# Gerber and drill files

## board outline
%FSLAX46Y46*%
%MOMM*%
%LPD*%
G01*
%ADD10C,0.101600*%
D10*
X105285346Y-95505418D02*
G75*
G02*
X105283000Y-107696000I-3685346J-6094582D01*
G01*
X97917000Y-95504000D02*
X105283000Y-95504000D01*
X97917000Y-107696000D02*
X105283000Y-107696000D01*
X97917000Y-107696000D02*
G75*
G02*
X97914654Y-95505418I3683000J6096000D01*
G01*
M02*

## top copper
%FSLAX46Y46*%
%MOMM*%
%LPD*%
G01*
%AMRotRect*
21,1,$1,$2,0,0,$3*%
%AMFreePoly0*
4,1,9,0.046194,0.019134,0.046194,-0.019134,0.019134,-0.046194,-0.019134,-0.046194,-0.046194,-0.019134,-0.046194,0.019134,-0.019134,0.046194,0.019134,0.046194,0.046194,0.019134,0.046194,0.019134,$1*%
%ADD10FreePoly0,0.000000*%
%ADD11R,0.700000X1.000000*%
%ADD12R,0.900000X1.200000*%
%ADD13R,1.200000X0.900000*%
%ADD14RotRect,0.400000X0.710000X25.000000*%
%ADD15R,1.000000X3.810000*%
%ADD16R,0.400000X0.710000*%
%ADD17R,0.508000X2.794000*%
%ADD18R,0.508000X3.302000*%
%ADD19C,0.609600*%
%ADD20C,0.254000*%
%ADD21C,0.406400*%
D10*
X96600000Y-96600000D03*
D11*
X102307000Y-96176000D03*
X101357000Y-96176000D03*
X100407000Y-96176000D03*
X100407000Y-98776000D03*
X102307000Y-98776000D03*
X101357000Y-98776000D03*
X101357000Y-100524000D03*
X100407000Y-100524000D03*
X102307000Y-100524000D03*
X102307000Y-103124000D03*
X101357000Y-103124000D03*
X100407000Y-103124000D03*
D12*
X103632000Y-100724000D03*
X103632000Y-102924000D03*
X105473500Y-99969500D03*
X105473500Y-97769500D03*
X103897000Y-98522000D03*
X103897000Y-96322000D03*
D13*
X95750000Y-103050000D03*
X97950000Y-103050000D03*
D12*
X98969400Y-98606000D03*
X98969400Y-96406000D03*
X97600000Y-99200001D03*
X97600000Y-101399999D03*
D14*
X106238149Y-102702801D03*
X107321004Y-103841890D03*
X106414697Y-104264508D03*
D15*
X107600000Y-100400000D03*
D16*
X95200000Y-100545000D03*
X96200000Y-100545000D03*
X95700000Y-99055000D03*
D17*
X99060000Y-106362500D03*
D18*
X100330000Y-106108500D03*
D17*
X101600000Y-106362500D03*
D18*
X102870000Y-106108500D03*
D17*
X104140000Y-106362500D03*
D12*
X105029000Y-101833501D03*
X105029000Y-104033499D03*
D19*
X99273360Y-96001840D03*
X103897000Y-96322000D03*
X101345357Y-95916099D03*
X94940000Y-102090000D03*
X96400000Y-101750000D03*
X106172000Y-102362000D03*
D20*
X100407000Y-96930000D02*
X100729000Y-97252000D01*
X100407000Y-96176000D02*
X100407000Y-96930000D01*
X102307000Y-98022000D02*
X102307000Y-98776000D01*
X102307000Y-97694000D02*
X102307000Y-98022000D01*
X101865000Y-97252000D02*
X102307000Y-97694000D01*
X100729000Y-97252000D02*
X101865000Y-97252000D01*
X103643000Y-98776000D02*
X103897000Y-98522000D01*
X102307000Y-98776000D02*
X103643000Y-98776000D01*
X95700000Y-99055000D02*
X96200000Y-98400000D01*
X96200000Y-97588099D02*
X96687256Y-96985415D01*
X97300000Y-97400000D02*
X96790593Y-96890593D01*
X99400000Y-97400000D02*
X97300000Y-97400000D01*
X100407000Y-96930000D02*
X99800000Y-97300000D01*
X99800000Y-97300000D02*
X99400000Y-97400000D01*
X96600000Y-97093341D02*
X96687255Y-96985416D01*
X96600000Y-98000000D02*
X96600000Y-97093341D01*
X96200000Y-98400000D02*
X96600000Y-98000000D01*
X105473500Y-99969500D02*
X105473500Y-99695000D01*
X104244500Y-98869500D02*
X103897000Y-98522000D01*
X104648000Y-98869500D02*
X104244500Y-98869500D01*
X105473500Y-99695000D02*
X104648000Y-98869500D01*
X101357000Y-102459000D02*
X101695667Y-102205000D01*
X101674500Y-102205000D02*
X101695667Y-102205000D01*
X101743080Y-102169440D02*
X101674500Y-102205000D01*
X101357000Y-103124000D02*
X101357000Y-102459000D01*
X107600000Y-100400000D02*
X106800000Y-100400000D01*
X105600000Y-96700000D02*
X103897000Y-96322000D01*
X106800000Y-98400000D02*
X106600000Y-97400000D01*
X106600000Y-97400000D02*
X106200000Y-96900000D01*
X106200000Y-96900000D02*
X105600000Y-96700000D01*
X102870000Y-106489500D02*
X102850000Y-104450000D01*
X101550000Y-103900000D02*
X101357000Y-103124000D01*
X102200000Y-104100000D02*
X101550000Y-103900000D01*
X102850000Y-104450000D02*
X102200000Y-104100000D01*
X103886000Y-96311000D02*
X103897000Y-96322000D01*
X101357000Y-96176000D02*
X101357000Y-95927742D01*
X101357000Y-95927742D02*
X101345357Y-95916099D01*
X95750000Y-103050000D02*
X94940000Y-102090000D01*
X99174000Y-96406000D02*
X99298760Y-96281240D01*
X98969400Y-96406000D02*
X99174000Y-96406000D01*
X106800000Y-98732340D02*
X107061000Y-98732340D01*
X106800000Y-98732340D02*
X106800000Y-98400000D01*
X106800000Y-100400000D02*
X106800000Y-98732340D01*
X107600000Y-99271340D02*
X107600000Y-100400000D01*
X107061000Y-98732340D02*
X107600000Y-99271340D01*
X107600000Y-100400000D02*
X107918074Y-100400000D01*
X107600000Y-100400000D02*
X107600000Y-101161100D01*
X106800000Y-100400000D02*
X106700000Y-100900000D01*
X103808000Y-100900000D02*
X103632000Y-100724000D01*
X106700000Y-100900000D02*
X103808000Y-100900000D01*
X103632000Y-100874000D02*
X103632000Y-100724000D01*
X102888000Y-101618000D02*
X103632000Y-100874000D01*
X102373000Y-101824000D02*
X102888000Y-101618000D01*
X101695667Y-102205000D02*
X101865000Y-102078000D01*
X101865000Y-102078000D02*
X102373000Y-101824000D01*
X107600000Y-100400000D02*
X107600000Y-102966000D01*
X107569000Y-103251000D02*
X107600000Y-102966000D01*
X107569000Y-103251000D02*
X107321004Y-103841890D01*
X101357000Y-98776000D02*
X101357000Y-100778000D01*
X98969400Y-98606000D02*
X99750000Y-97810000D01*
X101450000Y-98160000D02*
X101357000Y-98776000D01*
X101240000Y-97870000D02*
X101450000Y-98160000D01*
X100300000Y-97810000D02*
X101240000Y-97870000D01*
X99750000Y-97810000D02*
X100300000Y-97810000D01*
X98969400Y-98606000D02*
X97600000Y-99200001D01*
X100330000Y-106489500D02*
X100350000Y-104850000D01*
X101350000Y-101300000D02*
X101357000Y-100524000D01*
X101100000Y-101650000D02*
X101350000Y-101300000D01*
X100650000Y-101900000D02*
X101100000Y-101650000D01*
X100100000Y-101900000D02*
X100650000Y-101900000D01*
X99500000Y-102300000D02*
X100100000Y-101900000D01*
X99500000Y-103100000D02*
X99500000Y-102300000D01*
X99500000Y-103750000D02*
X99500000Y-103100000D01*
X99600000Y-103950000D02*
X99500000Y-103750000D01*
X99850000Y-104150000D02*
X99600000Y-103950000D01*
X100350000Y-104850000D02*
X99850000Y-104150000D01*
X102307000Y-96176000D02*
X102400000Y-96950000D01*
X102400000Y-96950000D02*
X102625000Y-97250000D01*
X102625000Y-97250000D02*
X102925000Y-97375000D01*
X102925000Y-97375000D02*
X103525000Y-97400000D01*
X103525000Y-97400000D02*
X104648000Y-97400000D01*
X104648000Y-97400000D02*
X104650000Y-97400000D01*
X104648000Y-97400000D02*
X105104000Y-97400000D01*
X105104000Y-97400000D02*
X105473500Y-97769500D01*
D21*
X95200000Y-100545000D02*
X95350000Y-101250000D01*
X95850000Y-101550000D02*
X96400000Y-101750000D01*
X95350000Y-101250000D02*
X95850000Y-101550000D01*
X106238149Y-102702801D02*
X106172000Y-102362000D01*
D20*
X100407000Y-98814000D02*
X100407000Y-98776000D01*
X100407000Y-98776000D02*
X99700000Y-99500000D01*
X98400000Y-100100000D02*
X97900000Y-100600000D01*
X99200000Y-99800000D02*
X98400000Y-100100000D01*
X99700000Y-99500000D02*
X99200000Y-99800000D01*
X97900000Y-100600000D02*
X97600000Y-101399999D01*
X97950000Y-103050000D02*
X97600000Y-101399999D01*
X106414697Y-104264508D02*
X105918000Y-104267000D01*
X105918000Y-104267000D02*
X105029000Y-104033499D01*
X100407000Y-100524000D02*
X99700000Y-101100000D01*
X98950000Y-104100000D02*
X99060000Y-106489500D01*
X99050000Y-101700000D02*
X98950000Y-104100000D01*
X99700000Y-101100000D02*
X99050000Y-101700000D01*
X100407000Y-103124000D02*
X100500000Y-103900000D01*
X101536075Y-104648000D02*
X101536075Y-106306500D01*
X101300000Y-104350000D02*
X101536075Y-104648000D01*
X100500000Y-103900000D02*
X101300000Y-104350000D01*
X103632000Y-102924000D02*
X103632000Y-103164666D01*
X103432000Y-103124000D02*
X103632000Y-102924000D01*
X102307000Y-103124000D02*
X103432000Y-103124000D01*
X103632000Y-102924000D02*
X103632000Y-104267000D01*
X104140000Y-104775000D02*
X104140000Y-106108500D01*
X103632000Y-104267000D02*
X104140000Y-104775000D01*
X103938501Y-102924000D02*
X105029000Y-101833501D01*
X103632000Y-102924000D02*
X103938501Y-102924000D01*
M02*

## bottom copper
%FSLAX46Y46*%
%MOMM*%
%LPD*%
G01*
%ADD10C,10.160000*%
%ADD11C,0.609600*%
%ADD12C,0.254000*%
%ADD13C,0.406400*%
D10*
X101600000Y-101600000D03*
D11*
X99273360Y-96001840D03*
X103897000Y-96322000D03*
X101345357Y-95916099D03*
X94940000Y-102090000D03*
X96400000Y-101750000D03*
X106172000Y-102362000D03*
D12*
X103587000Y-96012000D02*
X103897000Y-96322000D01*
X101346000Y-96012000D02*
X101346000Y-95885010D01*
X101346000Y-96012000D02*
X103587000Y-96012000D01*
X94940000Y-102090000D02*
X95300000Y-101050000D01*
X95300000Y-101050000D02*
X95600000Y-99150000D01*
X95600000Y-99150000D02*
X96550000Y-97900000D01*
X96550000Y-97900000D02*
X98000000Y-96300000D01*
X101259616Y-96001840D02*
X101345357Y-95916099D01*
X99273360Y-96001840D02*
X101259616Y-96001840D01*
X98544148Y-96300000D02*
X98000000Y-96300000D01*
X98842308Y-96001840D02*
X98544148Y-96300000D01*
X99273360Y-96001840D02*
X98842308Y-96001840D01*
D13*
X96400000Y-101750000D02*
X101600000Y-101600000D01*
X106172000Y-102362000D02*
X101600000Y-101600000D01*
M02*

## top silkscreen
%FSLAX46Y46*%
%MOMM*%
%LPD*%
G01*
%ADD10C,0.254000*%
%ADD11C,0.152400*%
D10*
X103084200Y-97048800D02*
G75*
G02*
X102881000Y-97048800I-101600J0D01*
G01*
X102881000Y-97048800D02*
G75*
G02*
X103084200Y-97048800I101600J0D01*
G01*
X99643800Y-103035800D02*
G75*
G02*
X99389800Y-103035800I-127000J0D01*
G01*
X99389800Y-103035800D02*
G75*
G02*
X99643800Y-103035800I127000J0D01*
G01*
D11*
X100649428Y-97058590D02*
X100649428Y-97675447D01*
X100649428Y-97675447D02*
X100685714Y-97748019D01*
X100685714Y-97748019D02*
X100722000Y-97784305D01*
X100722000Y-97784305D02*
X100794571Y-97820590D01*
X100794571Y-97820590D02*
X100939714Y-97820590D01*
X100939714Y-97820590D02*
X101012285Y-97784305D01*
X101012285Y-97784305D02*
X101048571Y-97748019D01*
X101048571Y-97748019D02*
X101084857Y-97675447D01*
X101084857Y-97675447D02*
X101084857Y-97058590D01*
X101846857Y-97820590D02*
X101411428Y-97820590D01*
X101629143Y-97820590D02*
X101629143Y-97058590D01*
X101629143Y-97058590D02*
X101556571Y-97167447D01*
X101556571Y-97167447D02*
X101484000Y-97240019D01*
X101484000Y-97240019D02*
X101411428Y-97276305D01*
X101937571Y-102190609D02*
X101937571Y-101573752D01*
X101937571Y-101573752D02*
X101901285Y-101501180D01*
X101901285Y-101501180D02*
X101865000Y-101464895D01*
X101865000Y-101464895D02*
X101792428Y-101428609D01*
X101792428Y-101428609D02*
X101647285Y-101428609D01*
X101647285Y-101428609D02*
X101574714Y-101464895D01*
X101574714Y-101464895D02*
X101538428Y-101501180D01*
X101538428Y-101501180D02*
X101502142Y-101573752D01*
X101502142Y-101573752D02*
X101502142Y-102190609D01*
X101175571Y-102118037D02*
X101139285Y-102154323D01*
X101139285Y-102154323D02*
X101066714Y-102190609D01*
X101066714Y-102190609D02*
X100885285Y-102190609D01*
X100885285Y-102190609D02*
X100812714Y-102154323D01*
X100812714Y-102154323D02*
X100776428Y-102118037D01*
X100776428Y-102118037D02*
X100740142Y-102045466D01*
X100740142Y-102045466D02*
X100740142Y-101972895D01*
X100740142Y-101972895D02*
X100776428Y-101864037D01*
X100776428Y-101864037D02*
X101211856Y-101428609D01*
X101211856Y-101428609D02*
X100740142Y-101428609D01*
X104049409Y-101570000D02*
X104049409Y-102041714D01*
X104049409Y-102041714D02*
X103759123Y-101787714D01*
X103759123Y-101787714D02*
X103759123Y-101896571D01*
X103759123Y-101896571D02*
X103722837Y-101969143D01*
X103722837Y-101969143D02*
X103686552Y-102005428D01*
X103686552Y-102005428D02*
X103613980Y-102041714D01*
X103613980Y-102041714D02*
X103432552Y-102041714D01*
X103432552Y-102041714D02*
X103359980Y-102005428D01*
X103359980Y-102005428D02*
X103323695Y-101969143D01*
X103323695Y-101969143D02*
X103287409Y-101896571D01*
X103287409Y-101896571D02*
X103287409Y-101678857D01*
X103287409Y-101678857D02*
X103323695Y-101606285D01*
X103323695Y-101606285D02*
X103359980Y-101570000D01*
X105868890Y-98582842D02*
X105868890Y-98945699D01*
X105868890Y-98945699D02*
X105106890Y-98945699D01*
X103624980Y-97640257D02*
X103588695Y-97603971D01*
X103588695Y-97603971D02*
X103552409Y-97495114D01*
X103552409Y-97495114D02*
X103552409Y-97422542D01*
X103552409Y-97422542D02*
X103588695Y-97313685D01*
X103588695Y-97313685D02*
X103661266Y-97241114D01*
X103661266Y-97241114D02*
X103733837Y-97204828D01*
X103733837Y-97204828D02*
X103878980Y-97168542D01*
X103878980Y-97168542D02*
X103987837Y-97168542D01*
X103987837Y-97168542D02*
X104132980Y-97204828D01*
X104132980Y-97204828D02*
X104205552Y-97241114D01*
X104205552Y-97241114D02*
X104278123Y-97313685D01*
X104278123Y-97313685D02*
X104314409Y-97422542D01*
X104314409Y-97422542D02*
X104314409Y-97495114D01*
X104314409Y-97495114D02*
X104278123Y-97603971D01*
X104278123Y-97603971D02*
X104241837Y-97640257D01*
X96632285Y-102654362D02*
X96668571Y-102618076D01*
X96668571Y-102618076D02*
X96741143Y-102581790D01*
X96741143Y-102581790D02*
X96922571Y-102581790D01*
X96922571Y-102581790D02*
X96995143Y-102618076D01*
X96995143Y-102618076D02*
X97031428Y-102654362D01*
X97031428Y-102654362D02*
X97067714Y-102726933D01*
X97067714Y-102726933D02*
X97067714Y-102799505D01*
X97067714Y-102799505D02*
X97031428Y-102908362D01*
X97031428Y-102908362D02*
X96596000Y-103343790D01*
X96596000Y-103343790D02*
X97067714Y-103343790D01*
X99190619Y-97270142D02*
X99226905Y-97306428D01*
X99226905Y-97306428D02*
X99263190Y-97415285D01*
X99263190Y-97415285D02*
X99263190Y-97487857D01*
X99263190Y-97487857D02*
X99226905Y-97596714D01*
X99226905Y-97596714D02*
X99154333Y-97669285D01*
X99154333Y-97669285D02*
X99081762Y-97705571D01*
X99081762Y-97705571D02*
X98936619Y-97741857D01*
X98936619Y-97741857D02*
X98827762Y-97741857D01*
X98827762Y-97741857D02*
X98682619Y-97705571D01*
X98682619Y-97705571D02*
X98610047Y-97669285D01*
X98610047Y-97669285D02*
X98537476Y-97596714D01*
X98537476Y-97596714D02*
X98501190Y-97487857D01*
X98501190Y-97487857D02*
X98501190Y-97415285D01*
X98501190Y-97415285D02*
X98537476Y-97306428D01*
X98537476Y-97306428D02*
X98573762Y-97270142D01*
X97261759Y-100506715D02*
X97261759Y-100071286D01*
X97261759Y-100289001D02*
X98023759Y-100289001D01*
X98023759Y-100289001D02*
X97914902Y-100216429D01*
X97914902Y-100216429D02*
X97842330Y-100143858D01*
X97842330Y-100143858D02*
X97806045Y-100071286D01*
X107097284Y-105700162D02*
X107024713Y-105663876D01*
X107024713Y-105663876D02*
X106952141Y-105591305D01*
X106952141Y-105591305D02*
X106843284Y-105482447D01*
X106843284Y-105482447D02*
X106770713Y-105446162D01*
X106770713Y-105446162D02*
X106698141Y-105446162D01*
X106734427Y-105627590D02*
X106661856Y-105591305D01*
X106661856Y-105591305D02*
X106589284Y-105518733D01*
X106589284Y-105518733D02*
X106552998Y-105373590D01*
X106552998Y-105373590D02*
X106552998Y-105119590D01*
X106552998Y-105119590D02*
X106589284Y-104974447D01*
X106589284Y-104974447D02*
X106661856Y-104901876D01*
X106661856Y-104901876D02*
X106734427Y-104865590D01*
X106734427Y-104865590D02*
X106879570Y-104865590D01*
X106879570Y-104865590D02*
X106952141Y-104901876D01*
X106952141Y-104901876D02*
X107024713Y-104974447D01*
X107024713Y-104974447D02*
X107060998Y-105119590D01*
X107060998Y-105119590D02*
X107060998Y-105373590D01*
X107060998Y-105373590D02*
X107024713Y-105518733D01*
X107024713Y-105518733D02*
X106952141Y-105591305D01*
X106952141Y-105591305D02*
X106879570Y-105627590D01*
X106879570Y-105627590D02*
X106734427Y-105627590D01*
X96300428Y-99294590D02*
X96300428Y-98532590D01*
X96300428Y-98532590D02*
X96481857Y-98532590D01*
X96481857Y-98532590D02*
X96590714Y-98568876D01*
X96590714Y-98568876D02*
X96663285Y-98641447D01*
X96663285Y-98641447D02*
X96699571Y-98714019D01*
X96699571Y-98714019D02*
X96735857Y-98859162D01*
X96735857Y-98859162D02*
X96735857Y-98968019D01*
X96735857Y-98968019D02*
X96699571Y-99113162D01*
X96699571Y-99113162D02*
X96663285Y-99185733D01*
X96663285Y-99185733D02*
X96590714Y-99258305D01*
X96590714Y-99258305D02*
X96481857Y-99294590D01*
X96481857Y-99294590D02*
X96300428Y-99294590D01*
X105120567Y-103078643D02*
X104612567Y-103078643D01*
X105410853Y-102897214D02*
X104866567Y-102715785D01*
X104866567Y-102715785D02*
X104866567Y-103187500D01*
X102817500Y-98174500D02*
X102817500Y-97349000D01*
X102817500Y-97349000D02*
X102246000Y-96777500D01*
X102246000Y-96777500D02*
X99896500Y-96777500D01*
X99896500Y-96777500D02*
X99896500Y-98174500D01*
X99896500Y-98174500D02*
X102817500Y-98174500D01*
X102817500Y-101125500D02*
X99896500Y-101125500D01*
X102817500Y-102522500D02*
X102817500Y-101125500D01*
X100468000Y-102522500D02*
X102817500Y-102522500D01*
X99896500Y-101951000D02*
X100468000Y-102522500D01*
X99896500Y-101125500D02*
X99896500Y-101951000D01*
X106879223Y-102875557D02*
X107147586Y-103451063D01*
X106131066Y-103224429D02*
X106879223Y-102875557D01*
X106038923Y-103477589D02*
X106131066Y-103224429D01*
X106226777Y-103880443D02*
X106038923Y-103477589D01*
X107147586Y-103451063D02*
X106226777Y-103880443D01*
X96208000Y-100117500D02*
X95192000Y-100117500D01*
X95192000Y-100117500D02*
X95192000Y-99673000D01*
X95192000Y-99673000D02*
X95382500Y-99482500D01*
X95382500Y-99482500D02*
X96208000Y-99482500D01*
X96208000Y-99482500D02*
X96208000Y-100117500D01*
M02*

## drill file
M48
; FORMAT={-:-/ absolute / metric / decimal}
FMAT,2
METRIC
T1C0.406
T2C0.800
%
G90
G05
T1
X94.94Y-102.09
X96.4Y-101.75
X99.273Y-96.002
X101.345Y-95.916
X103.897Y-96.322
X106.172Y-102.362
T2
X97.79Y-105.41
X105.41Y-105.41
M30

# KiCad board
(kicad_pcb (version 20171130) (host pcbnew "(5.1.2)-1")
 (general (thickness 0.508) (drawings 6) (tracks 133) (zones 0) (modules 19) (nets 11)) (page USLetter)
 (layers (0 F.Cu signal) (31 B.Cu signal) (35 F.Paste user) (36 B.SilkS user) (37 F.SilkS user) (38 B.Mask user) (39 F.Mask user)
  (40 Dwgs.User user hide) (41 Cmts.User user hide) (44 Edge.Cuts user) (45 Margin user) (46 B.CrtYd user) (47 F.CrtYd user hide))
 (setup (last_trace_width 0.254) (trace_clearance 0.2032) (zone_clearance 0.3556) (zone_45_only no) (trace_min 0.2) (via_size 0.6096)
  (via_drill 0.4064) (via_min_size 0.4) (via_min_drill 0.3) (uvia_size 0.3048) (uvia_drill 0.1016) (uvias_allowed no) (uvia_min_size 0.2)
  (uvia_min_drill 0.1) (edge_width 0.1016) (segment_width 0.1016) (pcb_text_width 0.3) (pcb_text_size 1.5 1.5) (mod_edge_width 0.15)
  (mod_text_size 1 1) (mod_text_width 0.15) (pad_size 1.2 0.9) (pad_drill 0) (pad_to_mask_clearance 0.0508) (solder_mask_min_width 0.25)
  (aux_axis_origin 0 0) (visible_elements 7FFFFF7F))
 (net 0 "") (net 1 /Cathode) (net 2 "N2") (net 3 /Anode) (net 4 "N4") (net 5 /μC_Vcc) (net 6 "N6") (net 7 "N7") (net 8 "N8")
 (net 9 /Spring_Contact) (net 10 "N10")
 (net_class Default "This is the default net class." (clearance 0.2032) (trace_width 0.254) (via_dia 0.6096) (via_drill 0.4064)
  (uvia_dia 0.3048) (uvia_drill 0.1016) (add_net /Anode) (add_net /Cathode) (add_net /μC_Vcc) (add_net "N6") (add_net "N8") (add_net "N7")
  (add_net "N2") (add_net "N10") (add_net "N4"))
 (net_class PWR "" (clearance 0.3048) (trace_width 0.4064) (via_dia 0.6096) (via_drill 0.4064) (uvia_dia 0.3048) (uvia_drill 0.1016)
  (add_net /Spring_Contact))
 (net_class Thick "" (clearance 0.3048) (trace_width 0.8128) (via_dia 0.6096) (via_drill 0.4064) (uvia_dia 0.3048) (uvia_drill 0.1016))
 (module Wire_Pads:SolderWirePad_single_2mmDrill (layer F.Cu) (at 105.41 105.41)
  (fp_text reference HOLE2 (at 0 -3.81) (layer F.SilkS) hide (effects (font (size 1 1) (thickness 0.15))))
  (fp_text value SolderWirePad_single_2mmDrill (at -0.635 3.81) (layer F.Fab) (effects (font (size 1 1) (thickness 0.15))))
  (pad "" np_thru_hole circle (at 0 0) (size 0.8 0.8) (drill 0.8) (layers *.Cu *.Mask)))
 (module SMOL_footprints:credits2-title (layer B.Cu) (at 101.6 101.727 100)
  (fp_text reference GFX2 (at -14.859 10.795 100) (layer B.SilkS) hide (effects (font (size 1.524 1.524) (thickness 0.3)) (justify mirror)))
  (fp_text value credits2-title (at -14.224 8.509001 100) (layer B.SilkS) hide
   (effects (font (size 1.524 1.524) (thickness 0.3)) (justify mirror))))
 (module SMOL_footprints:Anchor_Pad (layer F.Cu) (at 96.5 96.6)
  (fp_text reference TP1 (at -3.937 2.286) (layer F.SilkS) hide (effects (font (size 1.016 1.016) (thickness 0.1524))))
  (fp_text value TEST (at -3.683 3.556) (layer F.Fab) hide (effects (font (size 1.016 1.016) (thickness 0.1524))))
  (pad 1 smd custom (at 0.1 0) (size 0.1 0.1) (layers F.Cu F.Mask) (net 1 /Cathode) (zone_connect 0)
   (options (clearance outline) (anchor circle)) (primitives)))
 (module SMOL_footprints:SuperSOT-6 (layer F.Cu) (at 101.357 97.476 270)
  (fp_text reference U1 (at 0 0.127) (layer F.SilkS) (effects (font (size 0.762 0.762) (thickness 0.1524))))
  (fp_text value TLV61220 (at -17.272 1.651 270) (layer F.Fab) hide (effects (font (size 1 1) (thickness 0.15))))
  (fp_line (start 0.6985 -1.4605) (end -0.127 -1.4605) (layer F.SilkS) (width 0.1524))
  (fp_line (start -0.127 -1.4605) (end -0.6985 -0.889) (layer F.SilkS) (width 0.1524))
  (fp_line (start -0.6985 -0.889) (end -0.6985 1.4605) (layer F.SilkS) (width 0.1524))
  (fp_line (start -0.6985 1.4605) (end 0.6985 1.4605) (layer F.SilkS) (width 0.1524))
  (fp_line (start 0.6985 1.4605) (end 0.6985 -1.4605) (layer F.SilkS) (width 0.1524))
  (pad 1 smd rect (at -1.3 -0.95 270) (size 1 0.7) (layers F.Cu F.Paste F.Mask) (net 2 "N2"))
  (pad 2 smd rect (at -1.3 0 270) (size 1 0.7) (layers F.Cu F.Paste F.Mask) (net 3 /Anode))
  (pad 3 smd rect (at -1.3 0.95 270) (size 1 0.7) (layers F.Cu F.Paste F.Mask) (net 1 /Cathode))
  (pad 4 smd rect (at 1.3 0.95 270) (size 1 0.7) (layers F.Cu F.Paste F.Mask) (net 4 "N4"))
  (pad 6 smd rect (at 1.3 -0.95 270) (size 1 0.7) (layers F.Cu F.Paste F.Mask) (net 1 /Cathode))
  (pad 5 smd rect (at 1.3 0 270) (size 1 0.7) (layers F.Cu F.Paste F.Mask) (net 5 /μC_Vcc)))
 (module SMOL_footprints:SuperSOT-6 (layer F.Cu) (at 101.357 101.824 90)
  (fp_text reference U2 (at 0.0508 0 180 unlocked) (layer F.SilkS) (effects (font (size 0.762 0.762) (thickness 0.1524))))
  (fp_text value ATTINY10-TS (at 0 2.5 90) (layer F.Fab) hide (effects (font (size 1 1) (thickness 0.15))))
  (fp_line (start 0.6985 1.4605) (end 0.6985 -1.4605) (layer F.SilkS) (width 0.1524))
  (fp_line (start -0.6985 1.4605) (end 0.6985 1.4605) (layer F.SilkS) (width 0.1524))
  (fp_line (start -0.6985 -0.889) (end -0.6985 1.4605) (layer F.SilkS) (width 0.1524))
  (fp_line (start -0.127 -1.4605) (end -0.6985 -0.889) (layer F.SilkS) (width 0.1524))
  (fp_line (start 0.6985 -1.4605) (end -0.127 -1.4605) (layer F.SilkS) (width 0.1524))
  (pad 5 smd rect (at 1.3 0 90) (size 1 0.7) (layers F.Cu F.Paste F.Mask) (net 5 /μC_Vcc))
  (pad 6 smd rect (at 1.3 -0.95 90) (size 1 0.7) (layers F.Cu F.Paste F.Mask) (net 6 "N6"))
  (pad 4 smd rect (at 1.3 0.95 90) (size 1 0.7) (layers F.Cu F.Paste F.Mask))
  (pad 3 smd rect (at -1.3 0.95 90) (size 1 0.7) (layers F.Cu F.Paste F.Mask) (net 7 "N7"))
  (pad 2 smd rect (at -1.3 0 90) (size 1 0.7) (layers F.Cu F.Paste F.Mask) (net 3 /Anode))
  (pad 1 smd rect (at -1.3 -0.95 90) (size 1 0.7) (layers F.Cu F.Paste F.Mask) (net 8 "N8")))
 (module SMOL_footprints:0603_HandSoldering (layer F.Cu) (at 103.632 101.824 270)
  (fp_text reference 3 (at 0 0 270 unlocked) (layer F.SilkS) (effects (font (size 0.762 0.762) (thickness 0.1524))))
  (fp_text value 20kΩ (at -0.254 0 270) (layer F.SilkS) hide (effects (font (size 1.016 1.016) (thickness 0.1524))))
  (pad 1 smd rect (at -1.1 0 270) (size 1.2 0.9) (layers F.Cu F.Paste F.Mask) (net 3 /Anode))
  (pad 2 smd rect (at 1.1 0 270) (size 1.2 0.9) (layers F.Cu F.Paste F.Mask) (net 7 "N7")))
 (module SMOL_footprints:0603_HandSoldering (layer F.Cu) (at 105.4735 98.8695 90)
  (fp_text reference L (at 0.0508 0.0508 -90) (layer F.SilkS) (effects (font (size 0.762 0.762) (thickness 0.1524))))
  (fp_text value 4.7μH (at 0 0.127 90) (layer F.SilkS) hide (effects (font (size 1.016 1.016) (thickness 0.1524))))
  (pad 1 smd rect (at -1.1 0 90) (size 1.2 0.9) (layers F.Cu F.Paste F.Mask) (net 1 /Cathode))
  (pad 2 smd rect (at 1.1 0 90) (size 1.2 0.9) (layers F.Cu F.Paste F.Mask) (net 2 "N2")))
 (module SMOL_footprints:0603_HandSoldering (layer F.Cu) (at 103.897 97.422 90)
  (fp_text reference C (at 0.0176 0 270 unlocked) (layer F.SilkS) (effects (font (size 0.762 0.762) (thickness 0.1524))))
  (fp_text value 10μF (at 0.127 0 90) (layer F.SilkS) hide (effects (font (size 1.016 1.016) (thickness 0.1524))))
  (pad 1 smd rect (at -1.1 0 90) (size 1.2 0.9) (layers F.Cu F.Paste F.Mask) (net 1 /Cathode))
  (pad 2 smd rect (at 1.1 0 90) (size 1.2 0.9) (layers F.Cu F.Paste F.Mask) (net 3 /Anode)))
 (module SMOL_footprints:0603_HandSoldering (layer F.Cu) (at 96.85 103.05 180)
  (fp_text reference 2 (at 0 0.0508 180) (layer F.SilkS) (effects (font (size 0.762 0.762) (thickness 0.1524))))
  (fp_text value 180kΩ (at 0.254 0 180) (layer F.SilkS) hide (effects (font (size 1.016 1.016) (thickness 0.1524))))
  (pad 2 smd rect (at 1.1 0 180) (size 1.2 0.9) (layers F.Cu F.Paste F.Mask) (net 3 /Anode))
  (pad 1 smd rect (at -1.1 0 180) (size 1.2 0.9) (layers F.Cu F.Paste F.Mask) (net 4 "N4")))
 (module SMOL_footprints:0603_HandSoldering (layer F.Cu) (at 98.9694 97.506 90)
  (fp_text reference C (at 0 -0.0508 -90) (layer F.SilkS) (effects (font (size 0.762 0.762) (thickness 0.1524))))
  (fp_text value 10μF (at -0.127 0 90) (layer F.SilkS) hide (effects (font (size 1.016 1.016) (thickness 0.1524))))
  (pad 1 smd rect (at -1.1 0 90) (size 1.2 0.9) (layers F.Cu F.Paste F.Mask) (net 5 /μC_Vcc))
  (pad 2 smd rect (at 1.1 0 90) (size 1.2 0.9) (layers F.Cu F.Paste F.Mask) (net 3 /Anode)))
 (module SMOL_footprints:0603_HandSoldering (layer F.Cu) (at 97.6 100.3 270)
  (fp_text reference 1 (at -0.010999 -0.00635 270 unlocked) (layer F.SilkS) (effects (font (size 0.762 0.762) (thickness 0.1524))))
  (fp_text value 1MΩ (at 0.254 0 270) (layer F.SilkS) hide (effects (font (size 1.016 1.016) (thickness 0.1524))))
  (pad 1 smd rect (at -1.099999 0 270) (size 1.2 0.9) (layers F.Cu F.Paste F.Mask) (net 5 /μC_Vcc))
  (pad 2 smd rect (at 1.099999 0 270) (size 1.2 0.9) (layers F.Cu F.Paste F.Mask) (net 4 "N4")))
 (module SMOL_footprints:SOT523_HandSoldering (layer F.Cu) (at 106.553 103.378 25)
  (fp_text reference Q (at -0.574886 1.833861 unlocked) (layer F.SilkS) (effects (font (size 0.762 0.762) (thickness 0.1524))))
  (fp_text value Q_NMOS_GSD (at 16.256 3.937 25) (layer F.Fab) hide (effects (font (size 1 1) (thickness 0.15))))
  (fp_line (start 0.508 -0.3175) (end 0.508 0.3175) (layer F.SilkS) (width 0.1524))
  (fp_line (start -0.3175 -0.3175) (end 0.508 -0.3175) (layer F.SilkS) (width 0.1524))
  (fp_line (start -0.508 -0.127) (end -0.3175 -0.3175) (layer F.SilkS) (width 0.1524))
  (fp_line (start -0.508 0.3175) (end -0.508 -0.127) (layer F.SilkS) (width 0.1524))
  (fp_line (start 0.508 0.3175) (end -0.508 0.3175) (layer F.SilkS) (width 0.1524))
  (pad 3 smd rect (at 0 -0.745 25) (size 0.4 0.71) (layers F.Cu F.Paste F.Mask) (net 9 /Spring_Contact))
  (pad 2 smd rect (at 0.5 0.745 25) (size 0.4 0.71) (layers F.Cu F.Paste F.Mask) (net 3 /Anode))
  (pad 1 smd rect (at -0.5 0.745 25) (size 0.4 0.71) (layers F.Cu F.Paste F.Mask) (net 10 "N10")))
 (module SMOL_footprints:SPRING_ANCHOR (layer F.Cu) (at 107.6 100.4)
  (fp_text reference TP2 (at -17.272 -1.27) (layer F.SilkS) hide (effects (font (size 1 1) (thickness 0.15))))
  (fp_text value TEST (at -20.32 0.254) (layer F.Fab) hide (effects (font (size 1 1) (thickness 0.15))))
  (pad 1 smd rect (at 0 0) (size 1 3.81) (layers F.Cu F.Mask) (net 3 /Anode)))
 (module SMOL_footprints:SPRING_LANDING (layer B.Cu) (at 93.037 97.622)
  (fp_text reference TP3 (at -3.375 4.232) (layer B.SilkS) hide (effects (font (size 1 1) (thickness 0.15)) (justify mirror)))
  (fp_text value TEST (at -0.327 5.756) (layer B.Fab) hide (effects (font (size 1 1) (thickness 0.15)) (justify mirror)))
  (pad 1 smd circle (at 8.563 3.978) (size 10.16 10.16) (layers B.Cu B.Mask) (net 9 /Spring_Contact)))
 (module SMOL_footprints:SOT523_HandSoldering (layer F.Cu) (at 95.7 99.8)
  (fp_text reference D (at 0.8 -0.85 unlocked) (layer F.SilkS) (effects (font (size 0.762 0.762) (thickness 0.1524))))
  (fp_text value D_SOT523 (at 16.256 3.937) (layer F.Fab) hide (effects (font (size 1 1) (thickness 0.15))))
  (fp_line (start 0.508 0.3175) (end -0.508 0.3175) (layer F.SilkS) (width 0.1524))
  (fp_line (start -0.508 0.3175) (end -0.508 -0.127) (layer F.SilkS) (width 0.1524))
  (fp_line (start -0.508 -0.127) (end -0.3175 -0.3175) (layer F.SilkS) (width 0.1524))
  (fp_line (start -0.3175 -0.3175) (end 0.508 -0.3175) (layer F.SilkS) (width 0.1524))
  (fp_line (start 0.508 -0.3175) (end 0.508 0.3175) (layer F.SilkS) (width 0.1524))
  (pad 1 smd rect (at -0.5 0.745) (size 0.4 0.71) (layers F.Cu F.Paste F.Mask) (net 9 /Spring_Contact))
  (pad 2 smd rect (at 0.5 0.745) (size 0.4 0.71) (layers F.Cu F.Paste F.Mask))
  (pad 3 smd rect (at 0 -0.745) (size 0.4 0.71) (layers F.Cu F.Paste F.Mask) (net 1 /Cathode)))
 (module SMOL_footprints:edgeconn (layer F.Cu) (at 99.06 106.4895 90)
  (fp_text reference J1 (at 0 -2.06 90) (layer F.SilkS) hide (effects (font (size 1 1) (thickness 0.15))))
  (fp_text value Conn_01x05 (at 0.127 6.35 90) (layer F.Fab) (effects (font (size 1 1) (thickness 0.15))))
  (pad 1 smd rect (at 0.127 0 90) (size 2.794 0.508) (layers F.Cu F.Mask) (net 6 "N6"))
  (pad 2 smd rect (at 0.381 1.27 90) (size 3.302 0.508) (layers F.Cu F.Mask) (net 5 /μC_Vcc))
  (pad 3 smd rect (at 0.127 2.54 90) (size 2.794 0.508) (layers F.Cu F.Mask) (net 8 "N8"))
  (pad 4 smd rect (at 0.381 3.81 90) (size 3.302 0.508) (layers F.Cu F.Mask) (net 3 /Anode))
  (pad 5 smd rect (at 0.127 5.08 90) (size 2.794 0.508) (layers F.Cu F.Mask) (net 7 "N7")))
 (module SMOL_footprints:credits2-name (layer B.Cu) (at 101.6 101.6 258)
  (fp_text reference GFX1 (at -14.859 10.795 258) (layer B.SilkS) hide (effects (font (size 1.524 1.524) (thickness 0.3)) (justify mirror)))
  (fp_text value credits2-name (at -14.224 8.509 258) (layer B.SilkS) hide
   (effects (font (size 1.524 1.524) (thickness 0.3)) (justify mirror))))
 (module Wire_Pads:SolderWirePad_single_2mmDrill (layer F.Cu) (at 97.79 105.41)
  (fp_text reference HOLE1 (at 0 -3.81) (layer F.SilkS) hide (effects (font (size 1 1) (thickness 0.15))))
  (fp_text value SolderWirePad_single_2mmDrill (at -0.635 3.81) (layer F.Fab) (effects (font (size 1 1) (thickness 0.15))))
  (pad "" np_thru_hole circle (at 0 0) (size 0.8 0.8) (drill 0.8) (layers *.Cu *.Mask)))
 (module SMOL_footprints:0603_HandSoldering (layer F.Cu) (at 105.029 102.9335 270)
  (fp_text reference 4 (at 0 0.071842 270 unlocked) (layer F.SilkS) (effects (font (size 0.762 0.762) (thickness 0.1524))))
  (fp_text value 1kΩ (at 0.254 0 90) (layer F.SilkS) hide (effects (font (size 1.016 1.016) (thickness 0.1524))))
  (pad 1 smd rect (at -1.099999 0 270) (size 1.2 0.9) (layers F.Cu F.Paste F.Mask) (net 7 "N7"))
  (pad 2 smd rect (at 1.099999 0 270) (size 1.2 0.9) (layers F.Cu F.Paste F.Mask) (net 10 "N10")))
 (gr_arc (start 101.6 101.6) (end 105.283 107.696) (angle -117.7) (layer Edge.Cuts) (width 0.1016))
 (gr_line (start 97.917 95.504) (end 105.283 95.504) (angle 90) (layer Edge.Cuts) (width 0.1016))
 (gr_line (start 97.917 107.696) (end 105.283 107.696) (angle 90) (layer Edge.Cuts) (width 0.1016))
 (gr_circle (center 102.9826 97.0488) (end 102.9826 97.1504) (layer F.SilkS) (width 0.254))
 (gr_circle (center 99.5168 103.0358) (end 99.6438 103.0358) (layer F.SilkS) (width 0.254))
 (gr_arc (start 101.6 101.6) (end 97.917 107.696) (angle 117.7) (layer Edge.Cuts) (width 0.1016))
 (segment (start 100.407 96.93) (end 100.729 97.252) (width 0.254) (layer F.Cu) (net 1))
 (segment (start 100.407 96.176) (end 100.407 96.93) (width 0.254) (layer F.Cu) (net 1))
 (segment (start 102.307 98.022) (end 102.307 98.776) (width 0.254) (layer F.Cu) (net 1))
 (segment (start 102.307 97.694) (end 102.307 98.022) (width 0.254) (layer F.Cu) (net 1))
 (segment (start 101.865 97.252) (end 102.307 97.694) (width 0.254) (layer F.Cu) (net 1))
 (segment (start 100.729 97.252) (end 101.865 97.252) (width 0.254) (layer F.Cu) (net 1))
 (segment (start 103.643 98.776) (end 103.897 98.522) (width 0.254) (layer F.Cu) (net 1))
 (segment (start 102.307 98.776) (end 103.643 98.776) (width 0.254) (layer F.Cu) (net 1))
 (segment (start 95.7 99.055) (end 96.2 98.4) (width 0.254) (layer F.Cu) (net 1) (status 400000))
 (segment (start 96.2 97.588099) (end 96.687256 96.985415) (width 0.254) (layer F.Cu) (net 1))
 (segment (start 97.3 97.4) (end 96.790593 96.890593) (width 0.254) (layer F.Cu) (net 1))
 (segment (start 99.4 97.4) (end 97.3 97.4) (width 0.254) (layer F.Cu) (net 1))
 (segment (start 100.407 96.93) (end 99.8 97.3) (width 0.254) (layer F.Cu) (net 1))
 (segment (start 99.8 97.3) (end 99.4 97.4) (width 0.254) (layer F.Cu) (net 1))
 (segment (start 96.6 97.093341) (end 96.687255 96.985416) (width 0.254) (layer F.Cu) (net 1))
 (segment (start 96.6 98) (end 96.6 97.093341) (width 0.254) (layer F.Cu) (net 1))
 (segment (start 96.2 98.4) (end 96.6 98) (width 0.254) (layer F.Cu) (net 1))
 (segment (start 105.4735 99.9695) (end 105.4735 99.695) (width 0.254) (layer F.Cu) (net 1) (status C00000))
 (segment (start 104.2445 98.8695) (end 103.897 98.522) (width 0.254) (layer F.Cu) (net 1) (status C00000))
 (segment (start 104.648 98.8695) (end 104.2445 98.8695) (width 0.254) (layer F.Cu) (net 1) (status 800000))
 (segment (start 105.4735 99.695) (end 104.648 98.8695) (width 0.254) (layer F.Cu) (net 1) (status 400000))
 (segment (start 101.357 102.459) (end 101.695667 102.205) (width 0.254) (layer F.Cu) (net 3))
 (segment (start 101.6745 102.205) (end 101.695667 102.205) (width 0.254) (layer F.Cu) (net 3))
 (segment (start 101.74308 102.16944) (end 101.6745 102.205) (width 0.254) (layer F.Cu) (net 3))
 (segment (start 101.357 103.124) (end 101.357 102.459) (width 0.254) (layer F.Cu) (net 3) (status 400000))
 (segment (start 107.6 100.4) (end 106.8 100.4) (width 0.254) (layer F.Cu) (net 3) (status 400000))
 (segment (start 105.6 96.7) (end 103.897 96.322) (width 0.254) (layer F.Cu) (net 3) (status 800000))
 (segment (start 106.8 98.4) (end 106.6 97.4) (width 0.254) (layer F.Cu) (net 3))
 (segment (start 106.6 97.4) (end 106.2 96.9) (width 0.254) (layer F.Cu) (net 3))
 (segment (start 106.2 96.9) (end 105.6 96.7) (width 0.254) (layer F.Cu) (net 3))
 (segment (start 102.87 106.4895) (end 102.85 104.45) (width 0.254) (layer F.Cu) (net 3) (status 400000))
 (segment (start 101.55 103.9) (end 101.357 103.124) (width 0.254) (layer F.Cu) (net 3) (status 800000))
 (segment (start 102.2 104.1) (end 101.55 103.9) (width 0.254) (layer F.Cu) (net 3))
 (segment (start 102.85 104.45) (end 102.2 104.1) (width 0.254) (layer F.Cu) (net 3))
 (via (at 99.27336 96.00184) (size 0.6096) (drill 0.4064) (layers F.Cu B.Cu) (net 3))
 (segment (start 103.886 96.311) (end 103.897 96.322) (width 0.254) (layer F.Cu) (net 3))
 (via (at 103.897 96.322) (size 0.6096) (drill 0.4064) (layers F.Cu B.Cu) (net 3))
 (segment (start 103.587 96.012) (end 103.897 96.322) (width 0.254) (layer B.Cu) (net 3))
 (segment (start 101.346 96.012) (end 101.346 95.88501) (width 0.254) (layer B.Cu) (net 3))
 (segment (start 101.346 96.012) (end 103.587 96.012) (width 0.254) (layer B.Cu) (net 3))
 (via (at 101.345357 95.916099) (size 0.6096) (drill 0.4064) (layers F.Cu B.Cu) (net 3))
 (segment (start 101.357 96.176) (end 101.357 95.927742) (width 0.254) (layer F.Cu) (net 3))
 (segment (start 101.357 95.927742) (end 101.345357 95.916099) (width 0.254) (layer F.Cu) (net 3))
 (segment (start 95.75 103.05) (end 94.94 102.09) (width 0.254) (layer F.Cu) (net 3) (status 400000))
 (segment (start 94.94 102.09) (end 95.3 101.05) (width 0.254) (layer B.Cu) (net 3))
 (segment (start 95.3 101.05) (end 95.6 99.15) (width 0.254) (layer B.Cu) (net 3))
 (segment (start 95.6 99.15) (end 96.55 97.9) (width 0.254) (layer B.Cu) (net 3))
 (segment (start 96.55 97.9) (end 98 96.3) (width 0.254) (layer B.Cu) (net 3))
 (via (at 94.94 102.09) (size 0.6096) (drill 0.4064) (layers F.Cu B.Cu) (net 3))
 (segment (start 99.174 96.406) (end 99.29876 96.28124) (width 0.254) (layer F.Cu) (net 3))
 (segment (start 98.9694 96.406) (end 99.174 96.406) (width 0.254) (layer F.Cu) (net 3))
 (segment (start 101.259616 96.00184) (end 101.345357 95.916099) (width 0.254) (layer B.Cu) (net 3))
 (segment (start 99.27336 96.00184) (end 101.259616 96.00184) (width 0.254) (layer B.Cu) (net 3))
 (segment (start 98.544148 96.3) (end 98 96.3) (width 0.254) (layer B.Cu) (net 3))
 (segment (start 98.842308 96.00184) (end 98.544148 96.3) (width 0.254) (layer B.Cu) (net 3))
 (segment (start 99.27336 96.00184) (end 98.842308 96.00184) (width 0.254) (layer B.Cu) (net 3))
 (segment (start 106.8 98.73234) (end 107.061 98.73234) (width 0.254) (layer F.Cu) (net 3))
 (segment (start 106.8 98.73234) (end 106.8 98.4) (width 0.254) (layer F.Cu) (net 3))
 (segment (start 106.8 100.4) (end 106.8 98.73234) (width 0.254) (layer F.Cu) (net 3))
 (segment (start 107.6 99.27134) (end 107.6 100.4) (width 0.254) (layer F.Cu) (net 3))
 (segment (start 107.061 98.73234) (end 107.6 99.27134) (width 0.254) (layer F.Cu) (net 3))
 (segment (start 107.6 100.4) (end 107.918074 100.4) (width 0.254) (layer F.Cu) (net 3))
 (segment (start 107.6 100.4) (end 107.6 101.1611) (width 0.254) (layer F.Cu) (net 3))
 (segment (start 106.8 100.4) (end 106.7 100.9) (width 0.254) (layer F.Cu) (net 3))
 (segment (start 103.808 100.9) (end 103.632 100.724) (width 0.254) (layer F.Cu) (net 3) (status C00000))
 (segment (start 106.7 100.9) (end 103.808 100.9) (width 0.254) (layer F.Cu) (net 3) (status 800000))
 (segment (start 103.632 100.874) (end 103.632 100.724) (width 0.254) (layer F.Cu) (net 3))
 (segment (start 102.888 101.618) (end 103.632 100.874) (width 0.254) (layer F.Cu) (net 3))
 (segment (start 102.373 101.824) (end 102.888 101.618) (width 0.254) (layer F.Cu) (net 3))
 (segment (start 101.695667 102.205) (end 101.865 102.078) (width 0.254) (layer F.Cu) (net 3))
 (segment (start 101.865 102.078) (end 102.373 101.824) (width 0.254) (layer F.Cu) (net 3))
 (segment (start 107.6 100.4) (end 107.6 102.966) (width 0.254) (layer F.Cu) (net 3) (status 400000))
 (segment (start 107.569 103.251) (end 107.6 102.966) (width 0.254) (layer F.Cu) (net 3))
 (segment (start 107.569 103.251) (end 107.321004 103.84189) (width 0.254) (layer F.Cu) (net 3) (status 800000))
 (segment (start 101.357 98.776) (end 101.357 100.778) (width 0.254) (layer F.Cu) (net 5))
 (segment (start 98.9694 98.606) (end 99.75 97.81) (width 0.254) (layer F.Cu) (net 5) (status 400000))
 (segment (start 101.45 98.16) (end 101.357 98.776) (width 0.254) (layer F.Cu) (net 5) (status 800000))
 (segment (start 101.24 97.87) (end 101.45 98.16) (width 0.254) (layer F.Cu) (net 5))
 (segment (start 100.3 97.81) (end 101.24 97.87) (width 0.254) (layer F.Cu) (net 5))
 (segment (start 99.75 97.81) (end 100.3 97.81) (width 0.254) (layer F.Cu) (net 5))
 (segment (start 98.9694 98.606) (end 97.6 99.200001) (width 0.254) (layer F.Cu) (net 5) (status C00000))
 (segment (start 100.33 106.4895) (end 100.35 104.85) (width 0.254) (layer F.Cu) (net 5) (status 400000))
 (segment (start 101.35 101.3) (end 101.357 100.524) (width 0.254) (layer F.Cu) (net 5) (status 800000))
 (segment (start 101.1 101.65) (end 101.35 101.3) (width 0.254) (layer F.Cu) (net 5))
 (segment (start 100.65 101.9) (end 101.1 101.65) (width 0.254) (layer F.Cu) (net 5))
 (segment (start 100.1 101.9) (end 100.65 101.9) (width 0.254) (layer F.Cu) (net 5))
 (segment (start 99.5 102.3) (end 100.1 101.9) (width 0.254) (layer F.Cu) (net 5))
 (segment (start 99.5 103.1) (end 99.5 102.3) (width 0.254) (layer F.Cu) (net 5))
 (segment (start 99.5 103.75) (end 99.5 103.1) (width 0.254) (layer F.Cu) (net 5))
 (segment (start 99.6 103.95) (end 99.5 103.75) (width 0.254) (layer F.Cu) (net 5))
 (segment (start 99.85 104.15) (end 99.6 103.95) (width 0.254) (layer F.Cu) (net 5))
 (segment (start 100.35 104.85) (end 99.85 104.15) (width 0.254) (layer F.Cu) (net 5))
 (segment (start 102.307 96.176) (end 102.4 96.95) (width 0.254) (layer F.Cu) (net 2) (status 400000))
 (segment (start 102.4 96.95) (end 102.625 97.25) (width 0.254) (layer F.Cu) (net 2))
 (segment (start 102.625 97.25) (end 102.925 97.375) (width 0.254) (layer F.Cu) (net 2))
 (segment (start 102.925 97.375) (end 103.525 97.4) (width 0.254) (layer F.Cu) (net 2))
 (segment (start 103.525 97.4) (end 104.648 97.4) (width 0.254) (layer F.Cu) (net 2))
 (segment (start 104.648 97.4) (end 104.65 97.4) (width 0.254) (layer F.Cu) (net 2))
 (segment (start 104.648 97.4) (end 105.104 97.4) (width 0.254) (layer F.Cu) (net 2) (status 800000))
 (segment (start 105.104 97.4) (end 105.4735 97.7695) (width 0.254) (layer F.Cu) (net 2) (status C00000))
 (segment (start 95.2 100.545) (end 95.35 101.25) (width 0.4064) (layer F.Cu) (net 9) (status 400000))
 (segment (start 96.4 101.75) (end 101.6 101.6) (width 0.4064) (layer B.Cu) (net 9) (status 800000))
 (via (at 96.4 101.75) (size 0.6096) (drill 0.4064) (layers F.Cu B.Cu) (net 9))
 (segment (start 95.85 101.55) (end 96.4 101.75) (width 0.4064) (layer F.Cu) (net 9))
 (segment (start 95.35 101.25) (end 95.85 101.55) (width 0.4064) (layer F.Cu) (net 9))
 (segment (start 106.238149 102.702801) (end 106.172 102.362) (width 0.4064) (layer F.Cu) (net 9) (status C00000))
 (segment (start 106.172 102.362) (end 101.6 101.6) (width 0.4064) (layer B.Cu) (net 9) (status C00000))
 (via (at 106.172 102.362) (size 0.6096) (drill 0.4064) (layers F.Cu B.Cu) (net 9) (status C00000))
 (segment (start 100.407 98.814) (end 100.407 98.776) (width 0.254) (layer F.Cu) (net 4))
 (segment (start 100.407 98.776) (end 99.7 99.5) (width 0.254) (layer F.Cu) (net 4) (status 400000))
 (segment (start 98.4 100.1) (end 97.9 100.6) (width 0.254) (layer F.Cu) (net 4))
 (segment (start 99.2 99.8) (end 98.4 100.1) (width 0.254) (layer F.Cu) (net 4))
 (segment (start 99.7 99.5) (end 99.2 99.8) (width 0.254) (layer F.Cu) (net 4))
 (segment (start 97.9 100.6) (end 97.6 101.399999) (width 0.254) (layer F.Cu) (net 4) (status 800000))
 (segment (start 97.95 103.05) (end 97.6 101.399999) (width 0.254) (layer F.Cu) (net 4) (status C00000))
 (segment (start 106.414697 104.264508) (end 105.918 104.267) (width 0.254) (layer F.Cu) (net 10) (status 400000))
 (segment (start 105.918 104.267) (end 105.029 104.033499) (width 0.254) (layer F.Cu) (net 10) (status 800000))
 (segment (start 100.407 100.524) (end 99.7 101.1) (width 0.254) (layer F.Cu) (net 6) (status 400000))
 (segment (start 98.95 104.1) (end 99.06 106.4895) (width 0.254) (layer F.Cu) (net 6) (status 800000))
 (segment (start 99.05 101.7) (end 98.95 104.1) (width 0.254) (layer F.Cu) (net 6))
 (segment (start 99.7 101.1) (end 99.05 101.7) (width 0.254) (layer F.Cu) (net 6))
 (segment (start 100.407 103.124) (end 100.5 103.9) (width 0.254) (layer F.Cu) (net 8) (status 400000))
 (segment (start 101.536075 104.648) (end 101.536075 106.3065) (width 0.254) (layer F.Cu) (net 8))
 (segment (start 101.3 104.35) (end 101.536075 104.648) (width 0.254) (layer F.Cu) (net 8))
 (segment (start 100.5 103.9) (end 101.3 104.35) (width 0.254) (layer F.Cu) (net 8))
 (segment (start 103.632 102.924) (end 103.632 103.164666) (width 0.254) (layer F.Cu) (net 7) (status 400000))
 (segment (start 103.432 103.124) (end 103.632 102.924) (width 0.254) (layer F.Cu) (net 7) (status 800000))
 (segment (start 102.307 103.124) (end 103.432 103.124) (width 0.254) (layer F.Cu) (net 7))
 (segment (start 103.632 102.924) (end 103.632 104.267) (width 0.254) (layer F.Cu) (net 7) (status 400000))
 (segment (start 104.14 104.775) (end 104.14 106.1085) (width 0.254) (layer F.Cu) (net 7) (status C00000))
 (segment (start 103.632 104.267) (end 104.14 104.775) (width 0.254) (layer F.Cu) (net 7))
 (segment (start 103.938501 102.924) (end 105.029 101.833501) (width 0.254) (layer F.Cu) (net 7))
 (segment (start 103.632 102.924) (end 103.938501 102.924) (width 0.254) (layer F.Cu) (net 7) (status 400000)))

